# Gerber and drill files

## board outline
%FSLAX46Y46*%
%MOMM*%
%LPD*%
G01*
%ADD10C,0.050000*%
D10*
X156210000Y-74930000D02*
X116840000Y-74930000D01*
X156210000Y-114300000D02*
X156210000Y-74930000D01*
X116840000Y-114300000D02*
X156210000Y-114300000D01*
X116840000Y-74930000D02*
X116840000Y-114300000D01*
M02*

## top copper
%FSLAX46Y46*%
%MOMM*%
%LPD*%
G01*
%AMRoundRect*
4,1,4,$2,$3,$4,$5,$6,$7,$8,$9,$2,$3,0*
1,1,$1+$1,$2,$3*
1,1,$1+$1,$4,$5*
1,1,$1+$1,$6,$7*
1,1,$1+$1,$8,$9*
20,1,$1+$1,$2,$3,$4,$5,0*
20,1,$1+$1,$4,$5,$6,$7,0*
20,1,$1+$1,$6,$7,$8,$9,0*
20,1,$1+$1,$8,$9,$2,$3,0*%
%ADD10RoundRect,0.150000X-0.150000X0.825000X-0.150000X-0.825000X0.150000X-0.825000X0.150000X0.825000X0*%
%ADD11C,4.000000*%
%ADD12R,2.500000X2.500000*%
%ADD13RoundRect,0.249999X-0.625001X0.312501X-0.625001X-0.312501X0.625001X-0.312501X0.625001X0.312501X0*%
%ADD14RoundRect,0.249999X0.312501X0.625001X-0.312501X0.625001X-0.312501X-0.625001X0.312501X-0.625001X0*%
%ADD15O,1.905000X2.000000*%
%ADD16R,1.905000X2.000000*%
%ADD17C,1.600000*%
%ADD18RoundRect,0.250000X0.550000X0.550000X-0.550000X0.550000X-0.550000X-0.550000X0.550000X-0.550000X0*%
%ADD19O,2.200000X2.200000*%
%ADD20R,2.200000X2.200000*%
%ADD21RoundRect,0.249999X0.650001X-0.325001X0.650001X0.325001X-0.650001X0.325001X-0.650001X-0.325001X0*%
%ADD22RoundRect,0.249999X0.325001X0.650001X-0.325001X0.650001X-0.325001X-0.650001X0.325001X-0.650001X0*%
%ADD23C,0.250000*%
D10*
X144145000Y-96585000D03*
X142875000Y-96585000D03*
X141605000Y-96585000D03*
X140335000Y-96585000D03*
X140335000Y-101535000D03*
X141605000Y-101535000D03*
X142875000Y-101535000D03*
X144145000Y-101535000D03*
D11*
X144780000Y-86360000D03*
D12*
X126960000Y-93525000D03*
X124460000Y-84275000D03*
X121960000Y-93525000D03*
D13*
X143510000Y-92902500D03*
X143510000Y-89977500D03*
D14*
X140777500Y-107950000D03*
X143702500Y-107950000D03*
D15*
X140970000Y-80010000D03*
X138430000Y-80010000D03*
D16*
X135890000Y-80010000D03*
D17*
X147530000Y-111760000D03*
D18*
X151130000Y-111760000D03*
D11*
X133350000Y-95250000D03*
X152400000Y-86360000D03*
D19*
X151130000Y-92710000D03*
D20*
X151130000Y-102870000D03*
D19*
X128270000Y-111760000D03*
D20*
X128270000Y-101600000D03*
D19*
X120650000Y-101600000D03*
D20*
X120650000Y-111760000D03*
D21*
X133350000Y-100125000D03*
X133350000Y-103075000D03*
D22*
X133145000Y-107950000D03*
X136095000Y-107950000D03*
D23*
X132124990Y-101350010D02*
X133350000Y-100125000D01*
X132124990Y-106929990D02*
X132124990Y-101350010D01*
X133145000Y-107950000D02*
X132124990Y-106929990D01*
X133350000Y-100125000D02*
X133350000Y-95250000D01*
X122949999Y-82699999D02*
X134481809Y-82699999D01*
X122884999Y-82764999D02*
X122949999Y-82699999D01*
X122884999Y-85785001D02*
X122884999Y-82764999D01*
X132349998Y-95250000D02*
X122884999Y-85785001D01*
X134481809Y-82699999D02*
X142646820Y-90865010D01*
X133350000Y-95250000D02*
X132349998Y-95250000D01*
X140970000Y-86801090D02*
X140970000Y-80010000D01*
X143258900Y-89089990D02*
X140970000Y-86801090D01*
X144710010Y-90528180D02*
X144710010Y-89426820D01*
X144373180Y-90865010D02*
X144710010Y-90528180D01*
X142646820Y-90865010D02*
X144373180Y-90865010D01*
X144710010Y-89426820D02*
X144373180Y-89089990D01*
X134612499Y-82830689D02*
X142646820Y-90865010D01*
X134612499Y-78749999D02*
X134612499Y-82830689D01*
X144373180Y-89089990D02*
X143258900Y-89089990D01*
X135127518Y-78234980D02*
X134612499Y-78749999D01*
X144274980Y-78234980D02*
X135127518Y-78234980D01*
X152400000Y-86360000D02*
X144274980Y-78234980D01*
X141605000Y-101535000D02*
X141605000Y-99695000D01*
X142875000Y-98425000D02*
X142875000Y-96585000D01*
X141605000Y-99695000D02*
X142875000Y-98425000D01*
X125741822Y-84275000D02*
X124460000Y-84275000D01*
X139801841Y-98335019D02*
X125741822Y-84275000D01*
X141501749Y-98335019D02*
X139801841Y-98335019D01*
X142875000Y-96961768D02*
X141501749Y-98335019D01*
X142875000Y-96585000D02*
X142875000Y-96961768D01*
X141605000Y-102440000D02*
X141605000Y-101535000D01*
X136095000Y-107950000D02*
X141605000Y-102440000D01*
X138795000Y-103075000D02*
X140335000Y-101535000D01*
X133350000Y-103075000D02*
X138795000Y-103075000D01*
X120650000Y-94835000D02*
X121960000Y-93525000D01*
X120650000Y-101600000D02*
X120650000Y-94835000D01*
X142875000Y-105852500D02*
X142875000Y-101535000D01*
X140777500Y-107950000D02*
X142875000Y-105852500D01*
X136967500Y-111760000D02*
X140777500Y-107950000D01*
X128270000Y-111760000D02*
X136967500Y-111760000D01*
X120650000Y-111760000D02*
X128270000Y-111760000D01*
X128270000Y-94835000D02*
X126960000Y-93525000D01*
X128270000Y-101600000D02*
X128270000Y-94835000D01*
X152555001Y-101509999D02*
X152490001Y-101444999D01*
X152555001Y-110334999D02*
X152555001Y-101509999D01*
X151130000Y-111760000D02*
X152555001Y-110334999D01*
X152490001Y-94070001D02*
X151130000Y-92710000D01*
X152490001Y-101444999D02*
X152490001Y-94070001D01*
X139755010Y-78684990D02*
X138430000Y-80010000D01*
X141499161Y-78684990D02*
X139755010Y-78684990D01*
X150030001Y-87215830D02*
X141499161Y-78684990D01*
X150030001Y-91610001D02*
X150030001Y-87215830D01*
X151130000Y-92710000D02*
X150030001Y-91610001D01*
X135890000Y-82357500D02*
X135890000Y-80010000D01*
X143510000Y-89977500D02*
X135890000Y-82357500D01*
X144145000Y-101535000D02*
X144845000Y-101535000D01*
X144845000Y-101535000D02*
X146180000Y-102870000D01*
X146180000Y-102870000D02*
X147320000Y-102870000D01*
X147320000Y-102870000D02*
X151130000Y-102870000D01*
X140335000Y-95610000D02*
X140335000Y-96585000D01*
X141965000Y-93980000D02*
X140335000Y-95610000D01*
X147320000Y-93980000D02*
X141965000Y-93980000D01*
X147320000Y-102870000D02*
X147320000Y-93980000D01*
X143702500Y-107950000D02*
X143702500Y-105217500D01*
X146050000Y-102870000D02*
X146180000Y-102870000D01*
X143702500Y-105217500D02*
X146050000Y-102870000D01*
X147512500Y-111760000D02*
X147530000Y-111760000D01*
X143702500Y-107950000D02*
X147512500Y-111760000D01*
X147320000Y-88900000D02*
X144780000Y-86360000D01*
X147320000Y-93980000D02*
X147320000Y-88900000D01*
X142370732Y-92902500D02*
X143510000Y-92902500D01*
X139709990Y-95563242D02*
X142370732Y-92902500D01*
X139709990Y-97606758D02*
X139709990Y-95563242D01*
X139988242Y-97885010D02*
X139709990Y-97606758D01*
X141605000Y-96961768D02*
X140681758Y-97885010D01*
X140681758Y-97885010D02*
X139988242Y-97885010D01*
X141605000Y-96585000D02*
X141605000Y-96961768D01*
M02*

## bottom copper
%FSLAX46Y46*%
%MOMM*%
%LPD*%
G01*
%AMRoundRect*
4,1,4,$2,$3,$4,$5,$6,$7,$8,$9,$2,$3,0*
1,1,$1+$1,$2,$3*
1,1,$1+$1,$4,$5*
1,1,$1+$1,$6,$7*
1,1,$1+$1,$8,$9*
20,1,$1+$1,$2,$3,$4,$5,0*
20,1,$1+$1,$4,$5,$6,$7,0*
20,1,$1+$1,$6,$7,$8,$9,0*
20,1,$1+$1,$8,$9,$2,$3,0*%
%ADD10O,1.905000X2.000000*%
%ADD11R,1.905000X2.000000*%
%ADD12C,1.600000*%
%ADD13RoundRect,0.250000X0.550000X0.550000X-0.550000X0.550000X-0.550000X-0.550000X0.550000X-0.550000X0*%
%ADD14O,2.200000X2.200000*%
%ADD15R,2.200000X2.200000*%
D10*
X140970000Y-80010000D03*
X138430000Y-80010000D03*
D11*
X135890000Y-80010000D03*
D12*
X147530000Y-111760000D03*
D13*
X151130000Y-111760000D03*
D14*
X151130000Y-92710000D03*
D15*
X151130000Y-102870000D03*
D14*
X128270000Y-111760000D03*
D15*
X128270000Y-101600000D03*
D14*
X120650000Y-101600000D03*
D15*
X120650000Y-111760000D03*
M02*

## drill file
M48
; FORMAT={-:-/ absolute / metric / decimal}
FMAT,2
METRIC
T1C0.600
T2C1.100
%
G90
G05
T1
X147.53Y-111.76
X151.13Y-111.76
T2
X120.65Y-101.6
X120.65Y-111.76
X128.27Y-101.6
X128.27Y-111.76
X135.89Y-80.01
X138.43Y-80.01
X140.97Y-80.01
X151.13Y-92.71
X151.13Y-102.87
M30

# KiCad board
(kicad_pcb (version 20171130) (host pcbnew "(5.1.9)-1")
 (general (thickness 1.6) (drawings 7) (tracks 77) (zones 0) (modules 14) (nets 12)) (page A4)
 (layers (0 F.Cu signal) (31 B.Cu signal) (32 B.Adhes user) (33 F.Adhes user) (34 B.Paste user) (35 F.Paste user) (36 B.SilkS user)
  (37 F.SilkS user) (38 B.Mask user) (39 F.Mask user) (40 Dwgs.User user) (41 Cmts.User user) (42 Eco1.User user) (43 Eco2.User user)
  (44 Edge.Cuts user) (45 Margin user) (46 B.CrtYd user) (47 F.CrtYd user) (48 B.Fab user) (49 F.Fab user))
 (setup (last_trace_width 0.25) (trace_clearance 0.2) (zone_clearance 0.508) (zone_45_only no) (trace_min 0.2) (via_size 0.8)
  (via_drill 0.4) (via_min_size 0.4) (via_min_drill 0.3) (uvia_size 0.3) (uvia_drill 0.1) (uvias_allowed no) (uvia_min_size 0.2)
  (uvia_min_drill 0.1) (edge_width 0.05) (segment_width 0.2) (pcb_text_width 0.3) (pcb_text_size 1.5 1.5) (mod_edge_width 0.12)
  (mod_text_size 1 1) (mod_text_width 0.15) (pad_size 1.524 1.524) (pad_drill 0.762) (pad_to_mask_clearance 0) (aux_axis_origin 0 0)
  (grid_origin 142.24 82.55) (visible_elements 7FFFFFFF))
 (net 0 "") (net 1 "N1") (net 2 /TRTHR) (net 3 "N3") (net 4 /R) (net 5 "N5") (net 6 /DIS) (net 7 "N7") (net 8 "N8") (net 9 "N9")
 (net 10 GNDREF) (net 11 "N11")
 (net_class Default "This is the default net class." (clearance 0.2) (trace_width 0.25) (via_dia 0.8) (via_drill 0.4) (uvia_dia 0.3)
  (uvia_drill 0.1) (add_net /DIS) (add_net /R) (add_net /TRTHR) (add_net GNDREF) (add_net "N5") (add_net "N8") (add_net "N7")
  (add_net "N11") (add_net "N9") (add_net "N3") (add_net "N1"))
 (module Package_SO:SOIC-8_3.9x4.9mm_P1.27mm (layer F.Cu) (at 142.24 99.06 270)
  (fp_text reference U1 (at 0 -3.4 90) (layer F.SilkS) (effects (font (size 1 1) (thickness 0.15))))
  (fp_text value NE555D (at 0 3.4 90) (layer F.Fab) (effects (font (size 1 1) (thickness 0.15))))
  (pad 1 smd roundrect (at -2.475 -1.905 270) (size 1.95 0.6) (layers F.Cu F.Paste F.Mask) (roundrect_rratio 0.25) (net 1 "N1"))
  (pad 2 smd roundrect (at -2.475 -0.635 270) (size 1.95 0.6) (layers F.Cu F.Paste F.Mask) (roundrect_rratio 0.25) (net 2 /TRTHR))
  (pad 3 smd roundrect (at -2.475 0.635 270) (size 1.95 0.6) (layers F.Cu F.Paste F.Mask) (roundrect_rratio 0.25) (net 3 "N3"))
  (pad 4 smd roundrect (at -2.475 1.905 270) (size 1.95 0.6) (layers F.Cu F.Paste F.Mask) (roundrect_rratio 0.25) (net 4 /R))
  (pad 5 smd roundrect (at 2.475 1.905 270) (size 1.95 0.6) (layers F.Cu F.Paste F.Mask) (roundrect_rratio 0.25) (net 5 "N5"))
  (pad 6 smd roundrect (at 2.475 0.635 270) (size 1.95 0.6) (layers F.Cu F.Paste F.Mask) (roundrect_rratio 0.25) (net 2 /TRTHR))
  (pad 7 smd roundrect (at 2.475 -0.635 270) (size 1.95 0.6) (layers F.Cu F.Paste F.Mask) (roundrect_rratio 0.25) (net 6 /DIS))
  (pad 8 smd roundrect (at 2.475 -1.905 270) (size 1.95 0.6) (layers F.Cu F.Paste F.Mask) (roundrect_rratio 0.25) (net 4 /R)))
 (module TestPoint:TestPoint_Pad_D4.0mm (layer F.Cu) (at 144.78 86.36)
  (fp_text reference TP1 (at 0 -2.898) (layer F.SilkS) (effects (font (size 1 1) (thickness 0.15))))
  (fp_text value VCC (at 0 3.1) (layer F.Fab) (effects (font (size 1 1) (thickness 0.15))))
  (pad 1 smd circle (at 0 0) (size 4 4) (layers F.Cu F.Mask) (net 4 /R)))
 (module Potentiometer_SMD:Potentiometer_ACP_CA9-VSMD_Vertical (layer F.Cu) (at 124.46 88.9 90)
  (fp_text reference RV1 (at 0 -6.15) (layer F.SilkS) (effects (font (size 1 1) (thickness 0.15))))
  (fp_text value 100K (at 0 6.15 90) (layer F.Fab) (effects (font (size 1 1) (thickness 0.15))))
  (pad 1 smd rect (at -4.625 2.5 90) (size 2.5 2.5) (layers F.Cu F.Paste F.Mask) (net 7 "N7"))
  (pad 2 smd rect (at 4.625 0 90) (size 2.5 2.5) (layers F.Cu F.Paste F.Mask) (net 2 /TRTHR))
  (pad 3 smd rect (at -4.625 -2.5 90) (size 2.5 2.5) (layers F.Cu F.Paste F.Mask) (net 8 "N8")))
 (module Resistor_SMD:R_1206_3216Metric (layer F.Cu) (at 143.51 91.44 270)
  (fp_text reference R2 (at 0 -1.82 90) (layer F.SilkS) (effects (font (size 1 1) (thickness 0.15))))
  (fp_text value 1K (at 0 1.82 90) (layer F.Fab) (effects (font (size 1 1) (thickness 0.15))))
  (pad 2 smd roundrect (at 1.4625 0 270) (size 1.125 1.75) (layers F.Cu F.Paste F.Mask) (roundrect_rratio 0.2222213333333333) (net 3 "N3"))
  (pad 1 smd roundrect (at -1.4625 0 270) (size 1.125 1.75) (layers F.Cu F.Paste F.Mask) (roundrect_rratio 0.2222213333333333) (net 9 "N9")))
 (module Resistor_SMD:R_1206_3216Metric (layer F.Cu) (at 142.24 107.95 180)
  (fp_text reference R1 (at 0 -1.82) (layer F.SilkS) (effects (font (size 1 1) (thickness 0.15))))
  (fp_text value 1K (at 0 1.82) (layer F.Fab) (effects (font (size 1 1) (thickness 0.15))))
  (pad 2 smd roundrect (at 1.4625 0 180) (size 1.125 1.75) (layers F.Cu F.Paste F.Mask) (roundrect_rratio 0.2222213333333333) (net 6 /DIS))
  (pad 1 smd roundrect (at -1.4625 0 180) (size 1.125 1.75) (layers F.Cu F.Paste F.Mask) (roundrect_rratio 0.2222213333333333) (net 4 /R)))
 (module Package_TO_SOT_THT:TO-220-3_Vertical (layer F.Cu) (at 135.89 80.01)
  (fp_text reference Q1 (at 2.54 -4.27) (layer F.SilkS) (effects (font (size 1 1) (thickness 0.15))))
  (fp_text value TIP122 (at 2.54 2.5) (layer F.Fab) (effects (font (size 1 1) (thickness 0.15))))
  (pad 3 thru_hole oval (at 5.08 0) (size 1.905 2) (drill 1.1) (layers *.Cu *.Mask) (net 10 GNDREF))
  (pad 2 thru_hole oval (at 2.54 0) (size 1.905 2) (drill 1.1) (layers *.Cu *.Mask) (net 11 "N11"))
  (pad 1 thru_hole rect (at 0 0) (size 1.905 2) (drill 1.1) (layers *.Cu *.Mask) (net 9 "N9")))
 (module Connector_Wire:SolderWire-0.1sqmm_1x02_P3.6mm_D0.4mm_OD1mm (layer F.Cu) (at 151.13 111.76 180)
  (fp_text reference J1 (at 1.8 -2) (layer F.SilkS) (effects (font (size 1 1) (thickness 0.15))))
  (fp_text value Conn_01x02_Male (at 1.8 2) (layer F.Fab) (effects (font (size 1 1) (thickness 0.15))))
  (pad 2 thru_hole circle (at 3.6 0 180) (size 1.6 1.6) (drill 0.6) (layers *.Cu *.Mask) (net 4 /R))
  (pad 1 thru_hole roundrect (at 0 0 180) (size 1.6 1.6) (drill 0.6) (layers *.Cu *.Mask) (roundrect_rratio 0.15625) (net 11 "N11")))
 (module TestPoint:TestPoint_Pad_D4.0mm (layer F.Cu) (at 133.35 95.25)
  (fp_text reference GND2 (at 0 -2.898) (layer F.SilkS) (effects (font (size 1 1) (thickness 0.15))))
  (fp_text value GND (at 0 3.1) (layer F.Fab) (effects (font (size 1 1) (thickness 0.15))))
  (pad 1 smd circle (at 0 0) (size 4 4) (layers F.Cu F.Mask) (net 10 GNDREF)))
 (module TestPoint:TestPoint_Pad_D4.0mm (layer F.Cu) (at 152.4 86.36)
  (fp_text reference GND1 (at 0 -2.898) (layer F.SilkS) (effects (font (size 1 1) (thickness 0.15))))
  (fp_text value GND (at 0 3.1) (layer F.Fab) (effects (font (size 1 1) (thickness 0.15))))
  (pad 1 smd circle (at 0 0) (size 4 4) (layers F.Cu F.Mask) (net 10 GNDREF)))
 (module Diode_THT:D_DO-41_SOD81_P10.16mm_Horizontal (layer F.Cu) (at 151.13 102.87 90)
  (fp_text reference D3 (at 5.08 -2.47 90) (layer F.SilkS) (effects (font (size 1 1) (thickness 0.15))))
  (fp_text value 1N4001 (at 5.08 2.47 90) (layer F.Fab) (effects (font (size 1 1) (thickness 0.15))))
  (pad 2 thru_hole oval (at 10.16 0 90) (size 2.2 2.2) (drill 1.1) (layers *.Cu *.Mask) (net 11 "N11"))
  (pad 1 thru_hole rect (at 0 0 90) (size 2.2 2.2) (drill 1.1) (layers *.Cu *.Mask) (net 4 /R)))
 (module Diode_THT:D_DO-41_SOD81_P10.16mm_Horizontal (layer F.Cu) (at 128.27 101.6 270)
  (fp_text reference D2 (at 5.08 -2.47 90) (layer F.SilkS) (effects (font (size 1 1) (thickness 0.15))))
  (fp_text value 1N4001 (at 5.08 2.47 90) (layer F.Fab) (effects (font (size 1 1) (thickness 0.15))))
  (pad 2 thru_hole oval (at 10.16 0 270) (size 2.2 2.2) (drill 1.1) (layers *.Cu *.Mask) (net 6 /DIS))
  (pad 1 thru_hole rect (at 0 0 270) (size 2.2 2.2) (drill 1.1) (layers *.Cu *.Mask) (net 7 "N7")))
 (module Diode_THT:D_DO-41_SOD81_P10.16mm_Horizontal (layer F.Cu) (at 120.65 111.76 90)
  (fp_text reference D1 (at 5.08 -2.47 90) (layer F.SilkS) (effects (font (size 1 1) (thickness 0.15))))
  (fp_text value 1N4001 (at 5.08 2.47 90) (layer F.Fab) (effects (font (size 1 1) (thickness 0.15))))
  (pad 2 thru_hole oval (at 10.16 0 90) (size 2.2 2.2) (drill 1.1) (layers *.Cu *.Mask) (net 8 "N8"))
  (pad 1 thru_hole rect (at 0 0 90) (size 2.2 2.2) (drill 1.1) (layers *.Cu *.Mask) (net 6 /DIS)))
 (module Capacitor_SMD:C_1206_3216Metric (layer F.Cu) (at 133.35 101.6 90)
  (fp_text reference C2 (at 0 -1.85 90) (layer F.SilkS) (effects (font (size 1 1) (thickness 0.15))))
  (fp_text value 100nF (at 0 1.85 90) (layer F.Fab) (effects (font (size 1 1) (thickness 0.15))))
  (pad 2 smd roundrect (at 1.475 0 90) (size 1.15 1.8) (layers F.Cu F.Paste F.Mask) (roundrect_rratio 0.2173904347826087) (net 10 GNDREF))
  (pad 1 smd roundrect (at -1.475 0 90) (size 1.15 1.8) (layers F.Cu F.Paste F.Mask) (roundrect_rratio 0.2173904347826087) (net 5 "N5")))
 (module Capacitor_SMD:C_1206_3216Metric (layer F.Cu) (at 134.62 107.95 180)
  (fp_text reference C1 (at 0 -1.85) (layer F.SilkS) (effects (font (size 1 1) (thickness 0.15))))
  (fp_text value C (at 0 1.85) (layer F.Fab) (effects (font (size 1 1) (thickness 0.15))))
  (pad 2 smd roundrect (at 1.475 0 180) (size 1.15 1.8) (layers F.Cu F.Paste F.Mask) (roundrect_rratio 0.2173904347826087) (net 10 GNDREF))
  (pad 1 smd roundrect (at -1.475 0 180) (size 1.15 1.8) (layers F.Cu F.Paste F.Mask) (roundrect_rratio 0.2173904347826087) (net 2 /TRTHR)))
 (gr_line (start 156.21 74.93) (end 116.84 74.93) (layer Edge.Cuts) (width 0.05))
 (gr_line (start 156.21 114.3) (end 156.21 74.93) (layer Edge.Cuts) (width 0.05))
 (gr_line (start 116.84 114.3) (end 156.21 114.3) (layer Edge.Cuts) (width 0.05))
 (gr_line (start 116.84 74.93) (end 116.84 114.3) (layer Edge.Cuts) (width 0.05))
 (segment (start 132.12499 101.35001) (end 133.35 100.125) (width 0.25) (layer F.Cu) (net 10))
 (segment (start 132.12499 106.92999) (end 132.12499 101.35001) (width 0.25) (layer F.Cu) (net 10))
 (segment (start 133.145 107.95) (end 132.12499 106.92999) (width 0.25) (layer F.Cu) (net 10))
 (segment (start 133.35 100.125) (end 133.35 95.25) (width 0.25) (layer F.Cu) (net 10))
 (segment (start 122.949999 82.699999) (end 134.481809 82.699999) (width 0.25) (layer F.Cu) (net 10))
 (segment (start 122.884999 82.764999) (end 122.949999 82.699999) (width 0.25) (layer F.Cu) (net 10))
 (segment (start 122.884999 85.785001) (end 122.884999 82.764999) (width 0.25) (layer F.Cu) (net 10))
 (segment (start 132.349998 95.25) (end 122.884999 85.785001) (width 0.25) (layer F.Cu) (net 10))
 (segment (start 134.481809 82.699999) (end 142.64682 90.86501) (width 0.25) (layer F.Cu) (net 10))
 (segment (start 133.35 95.25) (end 132.349998 95.25) (width 0.25) (layer F.Cu) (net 10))
 (segment (start 140.97 86.80109) (end 140.97 80.01) (width 0.25) (layer F.Cu) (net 10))
 (segment (start 143.2589 89.08999) (end 140.97 86.80109) (width 0.25) (layer F.Cu) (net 10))
 (segment (start 144.71001 90.52818) (end 144.71001 89.42682) (width 0.25) (layer F.Cu) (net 10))
 (segment (start 144.37318 90.86501) (end 144.71001 90.52818) (width 0.25) (layer F.Cu) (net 10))
 (segment (start 142.64682 90.86501) (end 144.37318 90.86501) (width 0.25) (layer F.Cu) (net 10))
 (segment (start 144.71001 89.42682) (end 144.37318 89.08999) (width 0.25) (layer F.Cu) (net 10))
 (segment (start 134.612499 82.830689) (end 142.64682 90.86501) (width 0.25) (layer F.Cu) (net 10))
 (segment (start 134.612499 78.749999) (end 134.612499 82.830689) (width 0.25) (layer F.Cu) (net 10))
 (segment (start 144.37318 89.08999) (end 143.2589 89.08999) (width 0.25) (layer F.Cu) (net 10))
 (segment (start 135.127518 78.23498) (end 134.612499 78.749999) (width 0.25) (layer F.Cu) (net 10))
 (segment (start 144.27498 78.23498) (end 135.127518 78.23498) (width 0.25) (layer F.Cu) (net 10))
 (segment (start 152.4 86.36) (end 144.27498 78.23498) (width 0.25) (layer F.Cu) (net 10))
 (segment (start 141.605 101.535) (end 141.605 99.695) (width 0.25) (layer F.Cu) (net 2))
 (segment (start 142.875 98.425) (end 142.875 96.585) (width 0.25) (layer F.Cu) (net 2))
 (segment (start 141.605 99.695) (end 142.875 98.425) (width 0.25) (layer F.Cu) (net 2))
 (segment (start 125.741822 84.275) (end 124.46 84.275) (width 0.25) (layer F.Cu) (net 2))
 (segment (start 139.801841 98.335019) (end 125.741822 84.275) (width 0.25) (layer F.Cu) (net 2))
 (segment (start 141.501749 98.335019) (end 139.801841 98.335019) (width 0.25) (layer F.Cu) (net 2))
 (segment (start 142.875 96.961768) (end 141.501749 98.335019) (width 0.25) (layer F.Cu) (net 2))
 (segment (start 142.875 96.585) (end 142.875 96.961768) (width 0.25) (layer F.Cu) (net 2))
 (segment (start 141.605 102.44) (end 141.605 101.535) (width 0.25) (layer F.Cu) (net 2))
 (segment (start 136.095 107.95) (end 141.605 102.44) (width 0.25) (layer F.Cu) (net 2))
 (segment (start 138.795 103.075) (end 140.335 101.535) (width 0.25) (layer F.Cu) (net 5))
 (segment (start 133.35 103.075) (end 138.795 103.075) (width 0.25) (layer F.Cu) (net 5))
 (segment (start 120.65 94.835) (end 121.96 93.525) (width 0.25) (layer F.Cu) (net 8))
 (segment (start 120.65 101.6) (end 120.65 94.835) (width 0.25) (layer F.Cu) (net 8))
 (segment (start 142.875 105.8525) (end 142.875 101.535) (width 0.25) (layer F.Cu) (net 6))
 (segment (start 140.7775 107.95) (end 142.875 105.8525) (width 0.25) (layer F.Cu) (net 6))
 (segment (start 136.9675 111.76) (end 140.7775 107.95) (width 0.25) (layer F.Cu) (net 6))
 (segment (start 128.27 111.76) (end 136.9675 111.76) (width 0.25) (layer F.Cu) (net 6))
 (segment (start 120.65 111.76) (end 128.27 111.76) (width 0.25) (layer F.Cu) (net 6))
 (segment (start 128.27 94.835) (end 126.96 93.525) (width 0.25) (layer F.Cu) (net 7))
 (segment (start 128.27 101.6) (end 128.27 94.835) (width 0.25) (layer F.Cu) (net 7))
 (segment (start 152.555001 101.509999) (end 152.490001 101.444999) (width 0.25) (layer F.Cu) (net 11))
 (segment (start 152.555001 110.334999) (end 152.555001 101.509999) (width 0.25) (layer F.Cu) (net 11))
 (segment (start 151.13 111.76) (end 152.555001 110.334999) (width 0.25) (layer F.Cu) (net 11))
 (segment (start 152.490001 94.070001) (end 151.13 92.71) (width 0.25) (layer F.Cu) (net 11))
 (segment (start 152.490001 101.444999) (end 152.490001 94.070001) (width 0.25) (layer F.Cu) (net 11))
 (segment (start 139.75501 78.68499) (end 138.43 80.01) (width 0.25) (layer F.Cu) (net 11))
 (segment (start 141.499161 78.68499) (end 139.75501 78.68499) (width 0.25) (layer F.Cu) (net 11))
 (segment (start 150.030001 87.21583) (end 141.499161 78.68499) (width 0.25) (layer F.Cu) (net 11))
 (segment (start 150.030001 91.610001) (end 150.030001 87.21583) (width 0.25) (layer F.Cu) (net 11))
 (segment (start 151.13 92.71) (end 150.030001 91.610001) (width 0.25) (layer F.Cu) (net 11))
 (segment (start 135.89 82.3575) (end 135.89 80.01) (width 0.25) (layer F.Cu) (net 9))
 (segment (start 143.51 89.9775) (end 135.89 82.3575) (width 0.25) (layer F.Cu) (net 9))
 (segment (start 144.145 101.535) (end 144.845 101.535) (width 0.25) (layer F.Cu) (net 4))
 (segment (start 144.845 101.535) (end 146.18 102.87) (width 0.25) (layer F.Cu) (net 4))
 (segment (start 146.18 102.87) (end 147.32 102.87) (width 0.25) (layer F.Cu) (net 4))
 (segment (start 147.32 102.87) (end 151.13 102.87) (width 0.25) (layer F.Cu) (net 4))
 (segment (start 140.335 95.61) (end 140.335 96.585) (width 0.25) (layer F.Cu) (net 4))
 (segment (start 141.965 93.98) (end 140.335 95.61) (width 0.25) (layer F.Cu) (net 4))
 (segment (start 147.32 93.98) (end 141.965 93.98) (width 0.25) (layer F.Cu) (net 4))
 (segment (start 147.32 102.87) (end 147.32 93.98) (width 0.25) (layer F.Cu) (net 4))
 (segment (start 143.7025 107.95) (end 143.7025 105.2175) (width 0.25) (layer F.Cu) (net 4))
 (segment (start 146.05 102.87) (end 146.18 102.87) (width 0.25) (layer F.Cu) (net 4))
 (segment (start 143.7025 105.2175) (end 146.05 102.87) (width 0.25) (layer F.Cu) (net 4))
 (segment (start 147.5125 111.76) (end 147.53 111.76) (width 0.25) (layer F.Cu) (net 4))
 (segment (start 143.7025 107.95) (end 147.5125 111.76) (width 0.25) (layer F.Cu) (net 4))
 (segment (start 147.32 88.9) (end 144.78 86.36) (width 0.25) (layer F.Cu) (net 4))
 (segment (start 147.32 93.98) (end 147.32 88.9) (width 0.25) (layer F.Cu) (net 4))
 (segment (start 142.370732 92.9025) (end 143.51 92.9025) (width 0.25) (layer F.Cu) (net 3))
 (segment (start 139.70999 95.563242) (end 142.370732 92.9025) (width 0.25) (layer F.Cu) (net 3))
 (segment (start 139.70999 97.606758) (end 139.70999 95.563242) (width 0.25) (layer F.Cu) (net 3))
 (segment (start 139.988242 97.88501) (end 139.70999 97.606758) (width 0.25) (layer F.Cu) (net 3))
 (segment (start 141.605 96.961768) (end 140.681758 97.88501) (width 0.25) (layer F.Cu) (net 3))
 (segment (start 140.681758 97.88501) (end 139.988242 97.88501) (width 0.25) (layer F.Cu) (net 3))
 (segment (start 141.605 96.585) (end 141.605 96.961768) (width 0.25) (layer F.Cu) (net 3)))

